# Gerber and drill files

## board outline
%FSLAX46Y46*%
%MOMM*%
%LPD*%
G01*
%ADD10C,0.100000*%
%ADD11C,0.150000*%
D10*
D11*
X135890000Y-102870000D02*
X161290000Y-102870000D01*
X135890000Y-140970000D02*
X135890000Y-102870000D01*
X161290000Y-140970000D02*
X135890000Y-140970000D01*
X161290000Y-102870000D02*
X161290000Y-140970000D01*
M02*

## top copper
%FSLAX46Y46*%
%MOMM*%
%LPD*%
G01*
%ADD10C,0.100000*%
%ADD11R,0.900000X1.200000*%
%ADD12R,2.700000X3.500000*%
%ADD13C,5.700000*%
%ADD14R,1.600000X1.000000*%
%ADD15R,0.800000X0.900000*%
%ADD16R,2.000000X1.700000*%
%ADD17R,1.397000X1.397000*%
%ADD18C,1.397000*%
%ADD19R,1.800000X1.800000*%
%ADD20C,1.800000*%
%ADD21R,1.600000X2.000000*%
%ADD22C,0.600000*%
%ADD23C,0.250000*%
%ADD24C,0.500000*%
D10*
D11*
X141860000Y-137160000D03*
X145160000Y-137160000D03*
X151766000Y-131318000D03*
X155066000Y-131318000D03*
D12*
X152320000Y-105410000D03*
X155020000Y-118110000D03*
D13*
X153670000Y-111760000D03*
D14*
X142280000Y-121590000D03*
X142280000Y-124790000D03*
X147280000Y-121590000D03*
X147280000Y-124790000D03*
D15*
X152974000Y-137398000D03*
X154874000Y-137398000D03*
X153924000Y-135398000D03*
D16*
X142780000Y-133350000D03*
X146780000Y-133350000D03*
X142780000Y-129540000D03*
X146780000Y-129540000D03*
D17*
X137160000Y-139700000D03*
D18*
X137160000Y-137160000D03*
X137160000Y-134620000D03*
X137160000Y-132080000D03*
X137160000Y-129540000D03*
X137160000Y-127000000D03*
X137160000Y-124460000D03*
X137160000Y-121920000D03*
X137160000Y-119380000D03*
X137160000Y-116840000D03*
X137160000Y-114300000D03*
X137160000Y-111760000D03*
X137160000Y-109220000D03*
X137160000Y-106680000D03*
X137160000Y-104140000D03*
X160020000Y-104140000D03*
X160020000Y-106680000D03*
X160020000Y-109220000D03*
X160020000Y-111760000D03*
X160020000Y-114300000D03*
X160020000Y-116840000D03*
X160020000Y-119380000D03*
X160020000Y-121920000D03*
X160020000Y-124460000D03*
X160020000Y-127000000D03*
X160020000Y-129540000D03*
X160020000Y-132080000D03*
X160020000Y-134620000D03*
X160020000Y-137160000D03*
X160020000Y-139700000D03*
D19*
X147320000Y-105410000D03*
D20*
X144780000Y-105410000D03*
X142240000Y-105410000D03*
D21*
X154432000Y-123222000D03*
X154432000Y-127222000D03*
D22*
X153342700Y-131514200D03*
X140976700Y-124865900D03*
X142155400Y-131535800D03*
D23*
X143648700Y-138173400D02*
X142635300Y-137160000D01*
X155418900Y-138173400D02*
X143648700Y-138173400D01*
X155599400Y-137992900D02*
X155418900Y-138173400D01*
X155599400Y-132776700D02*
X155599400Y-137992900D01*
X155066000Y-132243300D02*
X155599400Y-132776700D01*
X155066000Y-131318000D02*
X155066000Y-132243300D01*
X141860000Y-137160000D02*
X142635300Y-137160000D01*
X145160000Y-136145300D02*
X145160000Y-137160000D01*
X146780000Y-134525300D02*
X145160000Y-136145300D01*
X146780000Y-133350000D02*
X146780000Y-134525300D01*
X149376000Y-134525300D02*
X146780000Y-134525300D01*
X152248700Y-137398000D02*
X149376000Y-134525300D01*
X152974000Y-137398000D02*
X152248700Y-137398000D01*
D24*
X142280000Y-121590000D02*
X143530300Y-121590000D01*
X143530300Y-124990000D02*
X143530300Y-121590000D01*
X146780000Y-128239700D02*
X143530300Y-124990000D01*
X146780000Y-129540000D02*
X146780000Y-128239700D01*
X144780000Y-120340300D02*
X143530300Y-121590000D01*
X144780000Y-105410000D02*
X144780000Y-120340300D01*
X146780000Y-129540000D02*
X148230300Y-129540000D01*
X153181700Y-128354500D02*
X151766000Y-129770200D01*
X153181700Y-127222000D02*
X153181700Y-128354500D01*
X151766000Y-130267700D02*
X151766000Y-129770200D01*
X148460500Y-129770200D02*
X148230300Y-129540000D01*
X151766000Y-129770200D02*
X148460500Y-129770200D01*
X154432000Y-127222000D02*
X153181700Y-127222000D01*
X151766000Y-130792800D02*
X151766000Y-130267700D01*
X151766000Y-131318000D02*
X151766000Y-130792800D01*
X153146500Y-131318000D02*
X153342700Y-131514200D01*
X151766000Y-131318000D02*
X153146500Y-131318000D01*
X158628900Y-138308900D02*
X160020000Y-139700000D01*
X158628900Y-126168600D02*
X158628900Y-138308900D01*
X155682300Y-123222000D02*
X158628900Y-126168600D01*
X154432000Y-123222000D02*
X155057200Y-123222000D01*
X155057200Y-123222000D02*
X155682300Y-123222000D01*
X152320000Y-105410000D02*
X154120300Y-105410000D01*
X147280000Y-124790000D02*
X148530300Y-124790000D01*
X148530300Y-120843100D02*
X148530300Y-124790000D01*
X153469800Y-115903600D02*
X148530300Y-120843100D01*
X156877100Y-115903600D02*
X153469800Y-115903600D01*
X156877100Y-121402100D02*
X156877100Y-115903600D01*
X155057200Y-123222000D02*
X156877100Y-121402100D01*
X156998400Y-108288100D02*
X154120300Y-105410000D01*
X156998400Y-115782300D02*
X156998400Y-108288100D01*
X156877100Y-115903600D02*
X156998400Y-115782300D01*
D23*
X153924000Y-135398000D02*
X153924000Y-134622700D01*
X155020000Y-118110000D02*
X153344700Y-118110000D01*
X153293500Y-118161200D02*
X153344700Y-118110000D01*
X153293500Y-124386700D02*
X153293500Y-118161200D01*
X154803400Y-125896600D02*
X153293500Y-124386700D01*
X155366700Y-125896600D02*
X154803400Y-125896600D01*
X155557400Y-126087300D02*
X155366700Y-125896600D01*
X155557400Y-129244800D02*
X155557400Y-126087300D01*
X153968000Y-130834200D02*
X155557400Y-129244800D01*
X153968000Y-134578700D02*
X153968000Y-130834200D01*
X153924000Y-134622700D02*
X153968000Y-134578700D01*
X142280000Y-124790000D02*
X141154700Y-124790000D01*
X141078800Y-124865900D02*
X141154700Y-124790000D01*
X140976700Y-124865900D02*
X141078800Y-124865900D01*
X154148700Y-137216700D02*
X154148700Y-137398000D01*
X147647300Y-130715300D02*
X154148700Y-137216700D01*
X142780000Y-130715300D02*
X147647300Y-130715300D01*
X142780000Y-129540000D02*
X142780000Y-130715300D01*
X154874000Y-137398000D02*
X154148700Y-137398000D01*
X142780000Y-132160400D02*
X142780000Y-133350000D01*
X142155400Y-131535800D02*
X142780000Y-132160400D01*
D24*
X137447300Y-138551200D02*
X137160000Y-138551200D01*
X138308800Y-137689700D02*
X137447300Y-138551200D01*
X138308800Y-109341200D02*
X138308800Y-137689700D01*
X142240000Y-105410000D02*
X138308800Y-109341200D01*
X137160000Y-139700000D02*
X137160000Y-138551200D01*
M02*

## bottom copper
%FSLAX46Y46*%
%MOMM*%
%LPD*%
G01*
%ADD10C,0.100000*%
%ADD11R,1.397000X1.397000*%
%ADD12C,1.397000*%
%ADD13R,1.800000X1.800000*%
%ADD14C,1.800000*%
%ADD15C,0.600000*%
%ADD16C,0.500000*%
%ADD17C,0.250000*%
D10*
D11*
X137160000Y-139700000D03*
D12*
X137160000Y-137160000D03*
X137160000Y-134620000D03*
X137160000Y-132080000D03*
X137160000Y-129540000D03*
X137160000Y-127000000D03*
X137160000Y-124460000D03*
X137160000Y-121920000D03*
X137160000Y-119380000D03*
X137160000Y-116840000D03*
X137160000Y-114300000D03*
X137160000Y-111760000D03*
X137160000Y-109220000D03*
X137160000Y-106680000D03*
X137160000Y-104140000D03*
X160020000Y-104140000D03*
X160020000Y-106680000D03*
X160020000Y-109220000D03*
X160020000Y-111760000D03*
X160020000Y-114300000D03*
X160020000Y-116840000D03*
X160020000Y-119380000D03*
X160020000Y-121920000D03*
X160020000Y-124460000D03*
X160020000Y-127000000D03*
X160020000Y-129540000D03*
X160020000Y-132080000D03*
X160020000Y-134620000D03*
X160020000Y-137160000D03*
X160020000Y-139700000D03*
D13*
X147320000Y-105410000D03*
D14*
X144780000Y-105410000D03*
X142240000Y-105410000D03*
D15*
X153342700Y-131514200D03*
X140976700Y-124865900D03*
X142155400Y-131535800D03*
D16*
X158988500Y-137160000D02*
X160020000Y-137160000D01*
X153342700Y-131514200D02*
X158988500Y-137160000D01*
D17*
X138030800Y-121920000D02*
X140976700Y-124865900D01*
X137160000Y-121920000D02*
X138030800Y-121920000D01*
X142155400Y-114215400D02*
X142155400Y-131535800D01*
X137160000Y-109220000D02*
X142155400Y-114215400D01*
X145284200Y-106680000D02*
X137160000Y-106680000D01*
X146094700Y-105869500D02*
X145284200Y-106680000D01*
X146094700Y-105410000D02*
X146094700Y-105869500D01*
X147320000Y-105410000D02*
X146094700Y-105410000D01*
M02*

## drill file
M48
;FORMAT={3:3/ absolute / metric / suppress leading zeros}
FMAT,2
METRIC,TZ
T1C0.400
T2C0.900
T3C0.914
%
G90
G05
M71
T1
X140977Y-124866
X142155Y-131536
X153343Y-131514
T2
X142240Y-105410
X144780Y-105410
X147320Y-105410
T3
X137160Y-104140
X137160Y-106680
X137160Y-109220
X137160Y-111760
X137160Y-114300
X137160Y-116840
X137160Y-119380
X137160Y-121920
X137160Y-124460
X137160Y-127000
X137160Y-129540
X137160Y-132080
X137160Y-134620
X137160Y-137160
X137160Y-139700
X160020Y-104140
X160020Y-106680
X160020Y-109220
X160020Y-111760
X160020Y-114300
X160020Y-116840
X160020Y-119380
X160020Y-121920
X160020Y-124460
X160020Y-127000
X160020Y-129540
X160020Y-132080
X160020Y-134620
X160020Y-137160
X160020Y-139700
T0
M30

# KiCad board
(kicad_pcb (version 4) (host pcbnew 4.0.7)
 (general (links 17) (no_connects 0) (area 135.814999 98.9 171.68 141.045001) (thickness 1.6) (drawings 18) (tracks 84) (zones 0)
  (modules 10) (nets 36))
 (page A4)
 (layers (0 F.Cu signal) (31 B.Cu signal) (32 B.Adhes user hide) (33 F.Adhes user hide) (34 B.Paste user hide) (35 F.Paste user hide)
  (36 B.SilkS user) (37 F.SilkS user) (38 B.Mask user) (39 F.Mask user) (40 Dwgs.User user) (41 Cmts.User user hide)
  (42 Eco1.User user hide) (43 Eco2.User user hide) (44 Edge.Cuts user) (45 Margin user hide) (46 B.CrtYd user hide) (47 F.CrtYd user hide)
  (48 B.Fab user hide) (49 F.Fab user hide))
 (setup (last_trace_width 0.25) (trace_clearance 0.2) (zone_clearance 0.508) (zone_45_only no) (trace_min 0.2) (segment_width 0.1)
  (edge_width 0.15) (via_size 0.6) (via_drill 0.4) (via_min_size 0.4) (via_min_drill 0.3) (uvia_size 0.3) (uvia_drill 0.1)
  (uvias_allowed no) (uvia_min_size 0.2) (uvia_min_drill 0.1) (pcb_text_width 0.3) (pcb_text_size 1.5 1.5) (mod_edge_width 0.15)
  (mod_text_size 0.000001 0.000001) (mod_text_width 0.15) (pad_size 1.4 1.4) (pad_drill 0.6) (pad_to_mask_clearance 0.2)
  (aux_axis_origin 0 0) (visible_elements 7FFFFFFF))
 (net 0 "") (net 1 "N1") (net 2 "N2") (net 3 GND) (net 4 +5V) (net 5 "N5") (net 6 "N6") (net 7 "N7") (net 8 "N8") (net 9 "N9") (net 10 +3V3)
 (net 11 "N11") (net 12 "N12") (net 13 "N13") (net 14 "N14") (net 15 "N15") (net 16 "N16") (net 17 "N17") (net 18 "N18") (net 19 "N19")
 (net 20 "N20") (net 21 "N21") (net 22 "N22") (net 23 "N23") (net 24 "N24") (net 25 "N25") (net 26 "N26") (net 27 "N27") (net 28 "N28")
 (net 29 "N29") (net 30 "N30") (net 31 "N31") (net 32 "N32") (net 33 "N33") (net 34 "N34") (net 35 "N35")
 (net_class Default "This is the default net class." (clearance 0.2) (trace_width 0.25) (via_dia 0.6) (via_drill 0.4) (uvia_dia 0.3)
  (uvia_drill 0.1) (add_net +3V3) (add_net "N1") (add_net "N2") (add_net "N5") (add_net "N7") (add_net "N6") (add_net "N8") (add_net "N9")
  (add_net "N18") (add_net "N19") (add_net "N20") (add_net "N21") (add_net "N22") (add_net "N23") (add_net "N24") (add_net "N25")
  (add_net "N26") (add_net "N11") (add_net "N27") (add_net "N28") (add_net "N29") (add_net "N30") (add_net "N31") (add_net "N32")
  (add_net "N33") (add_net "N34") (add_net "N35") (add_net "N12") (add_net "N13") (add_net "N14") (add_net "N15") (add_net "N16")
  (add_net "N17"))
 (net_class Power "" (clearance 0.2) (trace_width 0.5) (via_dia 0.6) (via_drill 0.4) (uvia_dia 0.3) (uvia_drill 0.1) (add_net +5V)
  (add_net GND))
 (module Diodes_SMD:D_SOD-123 (layer F.Cu) (at 143.51 137.16)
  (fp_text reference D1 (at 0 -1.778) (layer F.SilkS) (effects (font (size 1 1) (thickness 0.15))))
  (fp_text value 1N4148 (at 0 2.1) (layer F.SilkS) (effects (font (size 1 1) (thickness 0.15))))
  (pad 1 smd rect (at -1.65 0) (size 0.9 1.2) (layers F.Cu F.Paste F.Mask) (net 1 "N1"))
  (pad 2 smd rect (at 1.65 0) (size 0.9 1.2) (layers F.Cu F.Paste F.Mask) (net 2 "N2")))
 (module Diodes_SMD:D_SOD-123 (layer F.Cu) (at 153.416 131.318)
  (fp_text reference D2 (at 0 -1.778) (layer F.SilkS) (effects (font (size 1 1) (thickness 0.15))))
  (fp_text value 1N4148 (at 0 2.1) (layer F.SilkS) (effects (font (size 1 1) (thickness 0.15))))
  (pad 1 smd rect (at -1.65 0) (size 0.9 1.2) (layers F.Cu F.Paste F.Mask) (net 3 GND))
  (pad 2 smd rect (at 1.65 0) (size 0.9 1.2) (layers F.Cu F.Paste F.Mask) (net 1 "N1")))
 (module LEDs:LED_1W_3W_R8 (layer F.Cu) (at 153.67 111.76 90)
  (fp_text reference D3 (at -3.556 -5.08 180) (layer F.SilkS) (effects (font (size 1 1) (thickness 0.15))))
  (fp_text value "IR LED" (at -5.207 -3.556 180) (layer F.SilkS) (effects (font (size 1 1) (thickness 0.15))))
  (pad 2 smd rect (at 6.35 -1.35 90) (size 3.5 2.7) (layers F.Cu F.Paste F.Mask) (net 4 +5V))
  (pad 1 smd rect (at -6.35 1.35 90) (size 3.5 2.7) (layers F.Cu F.Paste F.Mask) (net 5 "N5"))
  (pad 3 smd circle (at 0 0 90) (size 5.7 5.7) (layers F.Cu F.Paste F.Mask)))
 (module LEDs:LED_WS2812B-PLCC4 (layer F.Cu) (at 144.78 123.19 180)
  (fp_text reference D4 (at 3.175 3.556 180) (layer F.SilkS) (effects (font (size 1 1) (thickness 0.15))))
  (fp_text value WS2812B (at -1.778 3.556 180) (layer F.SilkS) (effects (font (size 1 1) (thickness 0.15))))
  (pad 3 smd rect (at 2.5 1.6 180) (size 1.6 1) (layers F.Cu F.Paste F.Mask) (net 3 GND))
  (pad 4 smd rect (at 2.5 -1.6 180) (size 1.6 1) (layers F.Cu F.Paste F.Mask) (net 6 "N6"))
  (pad 2 smd rect (at -2.5 1.6 180) (size 1.6 1) (layers F.Cu F.Paste F.Mask) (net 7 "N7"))
  (pad 1 smd rect (at -2.5 -1.6 180) (size 1.6 1) (layers F.Cu F.Paste F.Mask) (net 4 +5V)))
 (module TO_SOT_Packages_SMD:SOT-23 (layer F.Cu) (at 153.924 136.398 90)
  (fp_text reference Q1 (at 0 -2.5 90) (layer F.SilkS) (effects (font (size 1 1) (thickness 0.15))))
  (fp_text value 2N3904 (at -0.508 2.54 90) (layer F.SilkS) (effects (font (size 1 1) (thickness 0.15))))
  (pad 1 smd rect (at -1 -0.95 90) (size 0.9 0.8) (layers F.Cu F.Paste F.Mask) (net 2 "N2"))
  (pad 2 smd rect (at -1 0.95 90) (size 0.9 0.8) (layers F.Cu F.Paste F.Mask) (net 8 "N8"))
  (pad 3 smd rect (at 1 0 90) (size 0.9 0.8) (layers F.Cu F.Paste F.Mask) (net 5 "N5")))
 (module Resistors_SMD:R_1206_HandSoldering (layer F.Cu) (at 144.78 133.35)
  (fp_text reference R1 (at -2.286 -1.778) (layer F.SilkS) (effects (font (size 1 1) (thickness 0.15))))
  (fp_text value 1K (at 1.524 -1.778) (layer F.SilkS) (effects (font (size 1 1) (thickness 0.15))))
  (pad 1 smd rect (at -2 0) (size 2 1.7) (layers F.Cu F.Paste F.Mask) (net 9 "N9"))
  (pad 2 smd rect (at 2 0) (size 2 1.7) (layers F.Cu F.Paste F.Mask) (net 2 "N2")))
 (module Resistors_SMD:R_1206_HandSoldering (layer F.Cu) (at 144.78 129.54)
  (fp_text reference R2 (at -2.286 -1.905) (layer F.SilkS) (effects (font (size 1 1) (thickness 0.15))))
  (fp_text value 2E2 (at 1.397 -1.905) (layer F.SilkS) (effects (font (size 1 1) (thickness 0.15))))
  (pad 1 smd rect (at -2 0) (size 2 1.7) (layers F.Cu F.Paste F.Mask) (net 8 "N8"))
  (pad 2 smd rect (at 2 0) (size 2 1.7) (layers F.Cu F.Paste F.Mask) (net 3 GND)))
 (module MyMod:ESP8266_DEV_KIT (layer B.Cu) (at 148.59 139.7)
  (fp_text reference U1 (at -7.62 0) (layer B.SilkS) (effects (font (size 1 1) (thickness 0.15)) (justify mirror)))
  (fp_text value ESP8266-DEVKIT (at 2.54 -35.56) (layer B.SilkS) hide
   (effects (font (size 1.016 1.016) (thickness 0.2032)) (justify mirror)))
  (pad 1 thru_hole rect (at -11.43 0) (size 1.397 1.397) (drill 0.9144) (layers *.Cu *.Mask B.SilkS) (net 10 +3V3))
  (pad 2 thru_hole circle (at -11.43 -2.54) (size 1.397 1.397) (drill 0.9144) (layers *.Cu *.Mask B.SilkS) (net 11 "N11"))
  (pad 3 thru_hole circle (at -11.43 -5.08) (size 1.397 1.397) (drill 0.9144) (layers *.Cu *.Mask B.SilkS) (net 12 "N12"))
  (pad 4 thru_hole circle (at -11.43 -7.62) (size 1.397 1.397) (drill 0.9144) (layers *.Cu *.Mask B.SilkS) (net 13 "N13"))
  (pad 5 thru_hole circle (at -11.43 -10.16) (size 1.397 1.397) (drill 0.9144) (layers *.Cu *.Mask B.SilkS) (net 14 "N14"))
  (pad 6 thru_hole circle (at -11.43 -12.7) (size 1.397 1.397) (drill 0.9144) (layers *.Cu *.Mask B.SilkS) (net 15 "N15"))
  (pad 7 thru_hole circle (at -11.43 -15.24) (size 1.397 1.397) (drill 0.9144) (layers *.Cu *.Mask B.SilkS) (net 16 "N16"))
  (pad 8 thru_hole circle (at -11.43 -17.78) (size 1.397 1.397) (drill 0.9144) (layers *.Cu *.Mask B.SilkS) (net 6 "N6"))
  (pad 9 thru_hole circle (at -11.43 -20.32) (size 1.397 1.397) (drill 0.9144) (layers *.Cu *.Mask B.SilkS) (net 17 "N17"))
  (pad 10 thru_hole circle (at -11.43 -22.86) (size 1.397 1.397) (drill 0.9144) (layers *.Cu *.Mask B.SilkS) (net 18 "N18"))
  (pad 11 thru_hole circle (at -11.43 -25.4) (size 1.397 1.397) (drill 0.9144) (layers *.Cu *.Mask B.SilkS) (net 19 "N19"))
  (pad 12 thru_hole circle (at -11.43 -27.94) (size 1.397 1.397) (drill 0.9144) (layers *.Cu *.Mask B.SilkS) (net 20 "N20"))
  (pad 13 thru_hole circle (at -11.43 -30.48) (size 1.397 1.397) (drill 0.9144) (layers *.Cu *.Mask B.SilkS) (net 9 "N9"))
  (pad 14 thru_hole circle (at -11.43 -33.02) (size 1.397 1.397) (drill 0.9144) (layers *.Cu *.Mask B.SilkS) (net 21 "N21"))
  (pad 15 thru_hole circle (at -11.43 -35.56) (size 1.397 1.397) (drill 0.9144) (layers *.Cu *.Mask B.SilkS) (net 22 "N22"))
  (pad 16 thru_hole circle (at 11.43 -35.56) (size 1.397 1.397) (drill 0.9144) (layers *.Cu *.Mask B.SilkS) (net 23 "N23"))
  (pad 17 thru_hole circle (at 11.43 -33.02) (size 1.397 1.397) (drill 0.9144) (layers *.Cu *.Mask B.SilkS) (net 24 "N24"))
  (pad 18 thru_hole circle (at 11.43 -30.48) (size 1.397 1.397) (drill 0.9144) (layers *.Cu *.Mask B.SilkS) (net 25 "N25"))
  (pad 19 thru_hole circle (at 11.43 -27.94) (size 1.397 1.397) (drill 0.9144) (layers *.Cu *.Mask B.SilkS) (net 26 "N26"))
  (pad 20 thru_hole circle (at 11.43 -25.4) (size 1.397 1.397) (drill 0.9144) (layers *.Cu *.Mask B.SilkS) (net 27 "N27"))
  (pad 21 thru_hole circle (at 11.43 -22.86) (size 1.397 1.397) (drill 0.9144) (layers *.Cu *.Mask B.SilkS) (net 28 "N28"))
  (pad 22 thru_hole circle (at 11.43 -20.32) (size 1.397 1.397) (drill 0.9144) (layers *.Cu *.Mask B.SilkS) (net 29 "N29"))
  (pad 23 thru_hole circle (at 11.43 -17.78) (size 1.397 1.397) (drill 0.9144) (layers *.Cu *.Mask B.SilkS) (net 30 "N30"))
  (pad 24 thru_hole circle (at 11.43 -15.24) (size 1.397 1.397) (drill 0.9144) (layers *.Cu *.Mask B.SilkS) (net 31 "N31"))
  (pad 25 thru_hole circle (at 11.43 -12.7) (size 1.397 1.397) (drill 0.9144) (layers *.Cu *.Mask B.SilkS) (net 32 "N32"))
  (pad 26 thru_hole circle (at 11.43 -10.16) (size 1.397 1.397) (drill 0.9144) (layers *.Cu *.Mask B.SilkS) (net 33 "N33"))
  (pad 27 thru_hole circle (at 11.43 -7.62) (size 1.397 1.397) (drill 0.9144) (layers *.Cu *.Mask B.SilkS) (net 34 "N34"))
  (pad 28 thru_hole circle (at 11.43 -5.08) (size 1.397 1.397) (drill 0.9144) (layers *.Cu *.Mask B.SilkS) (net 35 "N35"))
  (pad 29 thru_hole circle (at 11.43 -2.54) (size 1.397 1.397) (drill 0.9144) (layers *.Cu *.Mask B.SilkS) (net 3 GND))
  (pad 30 thru_hole circle (at 11.43 0) (size 1.397 1.397) (drill 0.9144) (layers *.Cu *.Mask B.SilkS) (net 4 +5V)))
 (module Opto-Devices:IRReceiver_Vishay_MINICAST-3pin (layer F.Cu) (at 147.32 105.41 180)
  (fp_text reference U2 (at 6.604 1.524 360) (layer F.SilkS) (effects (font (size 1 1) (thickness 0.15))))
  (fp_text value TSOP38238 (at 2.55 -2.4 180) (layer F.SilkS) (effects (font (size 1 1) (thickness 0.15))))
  (pad 1 thru_hole rect (at 0 0 180) (size 1.8 1.8) (drill 0.9) (layers *.Cu *.Mask) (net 21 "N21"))
  (pad 2 thru_hole circle (at 2.54 0 180) (size 1.8 1.8) (drill 0.9) (layers *.Cu *.Mask) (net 3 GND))
  (pad 3 thru_hole circle (at 5.08 0 180) (size 1.8 1.8) (drill 0.9) (layers *.Cu *.Mask) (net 10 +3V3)))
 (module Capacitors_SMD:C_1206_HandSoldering (layer F.Cu) (at 154.432 125.222 270)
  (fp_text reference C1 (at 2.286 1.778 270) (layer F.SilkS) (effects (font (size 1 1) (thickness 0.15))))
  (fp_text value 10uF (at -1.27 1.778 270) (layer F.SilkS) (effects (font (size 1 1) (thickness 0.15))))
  (pad 1 smd rect (at -2 0 270) (size 2 1.6) (layers F.Cu F.Paste F.Mask) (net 4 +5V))
  (pad 2 smd rect (at 2 0 270) (size 2 1.6) (layers F.Cu F.Paste F.Mask) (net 3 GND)))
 (gr_line (start 135.89 102.87) (end 161.29 102.87) (angle 90) (layer Edge.Cuts) (width 0.15))
 (gr_line (start 135.89 140.97) (end 135.89 102.87) (angle 90) (layer Edge.Cuts) (width 0.15))
 (gr_line (start 161.29 140.97) (end 135.89 140.97) (angle 90) (layer Edge.Cuts) (width 0.15))
 (gr_line (start 161.29 102.87) (end 161.29 140.97) (angle 90) (layer Edge.Cuts) (width 0.15))
 (segment (start 143.6487 138.1734) (end 142.6353 137.16) (width 0.25) (layer F.Cu) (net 1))
 (segment (start 155.4189 138.1734) (end 143.6487 138.1734) (width 0.25) (layer F.Cu) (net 1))
 (segment (start 155.5994 137.9929) (end 155.4189 138.1734) (width 0.25) (layer F.Cu) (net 1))
 (segment (start 155.5994 132.7767) (end 155.5994 137.9929) (width 0.25) (layer F.Cu) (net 1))
 (segment (start 155.066 132.2433) (end 155.5994 132.7767) (width 0.25) (layer F.Cu) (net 1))
 (segment (start 155.066 131.318) (end 155.066 132.2433) (width 0.25) (layer F.Cu) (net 1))
 (segment (start 141.86 137.16) (end 142.6353 137.16) (width 0.25) (layer F.Cu) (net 1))
 (segment (start 145.16 136.1453) (end 145.16 137.16) (width 0.25) (layer F.Cu) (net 2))
 (segment (start 146.78 134.5253) (end 145.16 136.1453) (width 0.25) (layer F.Cu) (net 2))
 (segment (start 146.78 133.35) (end 146.78 134.5253) (width 0.25) (layer F.Cu) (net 2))
 (segment (start 149.376 134.5253) (end 146.78 134.5253) (width 0.25) (layer F.Cu) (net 2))
 (segment (start 152.2487 137.398) (end 149.376 134.5253) (width 0.25) (layer F.Cu) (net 2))
 (segment (start 152.974 137.398) (end 152.2487 137.398) (width 0.25) (layer F.Cu) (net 2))
 (via (at 153.3427 131.5142) (size 0.6) (layers F.Cu B.Cu) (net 3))
 (segment (start 142.28 121.59) (end 143.5303 121.59) (width 0.5) (layer F.Cu) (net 3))
 (segment (start 143.5303 124.99) (end 143.5303 121.59) (width 0.5) (layer F.Cu) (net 3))
 (segment (start 146.78 128.2397) (end 143.5303 124.99) (width 0.5) (layer F.Cu) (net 3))
 (segment (start 146.78 129.54) (end 146.78 128.2397) (width 0.5) (layer F.Cu) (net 3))
 (segment (start 144.78 120.3403) (end 143.5303 121.59) (width 0.5) (layer F.Cu) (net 3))
 (segment (start 144.78 105.41) (end 144.78 120.3403) (width 0.5) (layer F.Cu) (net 3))
 (segment (start 146.78 129.54) (end 148.2303 129.54) (width 0.5) (layer F.Cu) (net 3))
 (segment (start 153.1817 128.3545) (end 151.766 129.7702) (width 0.5) (layer F.Cu) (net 3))
 (segment (start 153.1817 127.222) (end 153.1817 128.3545) (width 0.5) (layer F.Cu) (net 3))
 (segment (start 151.766 130.2677) (end 151.766 129.7702) (width 0.5) (layer F.Cu) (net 3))
 (segment (start 148.4605 129.7702) (end 148.2303 129.54) (width 0.5) (layer F.Cu) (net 3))
 (segment (start 151.766 129.7702) (end 148.4605 129.7702) (width 0.5) (layer F.Cu) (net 3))
 (segment (start 154.432 127.222) (end 153.1817 127.222) (width 0.5) (layer F.Cu) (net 3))
 (segment (start 151.766 130.7928) (end 151.766 130.2677) (width 0.5) (layer F.Cu) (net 3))
 (segment (start 158.9885 137.16) (end 160.02 137.16) (width 0.5) (layer B.Cu) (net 3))
 (segment (start 153.3427 131.5142) (end 158.9885 137.16) (width 0.5) (layer B.Cu) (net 3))
 (segment (start 151.766 131.318) (end 151.766 130.7928) (width 0.5) (layer F.Cu) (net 3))
 (segment (start 153.1465 131.318) (end 153.3427 131.5142) (width 0.5) (layer F.Cu) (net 3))
 (segment (start 151.766 131.318) (end 153.1465 131.318) (width 0.5) (layer F.Cu) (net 3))
 (segment (start 158.6289 138.3089) (end 160.02 139.7) (width 0.5) (layer F.Cu) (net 4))
 (segment (start 158.6289 126.1686) (end 158.6289 138.3089) (width 0.5) (layer F.Cu) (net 4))
 (segment (start 155.6823 123.222) (end 158.6289 126.1686) (width 0.5) (layer F.Cu) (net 4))
 (segment (start 154.432 123.222) (end 155.0572 123.222) (width 0.5) (layer F.Cu) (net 4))
 (segment (start 155.0572 123.222) (end 155.6823 123.222) (width 0.5) (layer F.Cu) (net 4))
 (segment (start 152.32 105.41) (end 154.1203 105.41) (width 0.5) (layer F.Cu) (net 4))
 (segment (start 147.28 124.79) (end 148.5303 124.79) (width 0.5) (layer F.Cu) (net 4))
 (segment (start 148.5303 120.8431) (end 148.5303 124.79) (width 0.5) (layer F.Cu) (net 4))
 (segment (start 153.4698 115.9036) (end 148.5303 120.8431) (width 0.5) (layer F.Cu) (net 4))
 (segment (start 156.8771 115.9036) (end 153.4698 115.9036) (width 0.5) (layer F.Cu) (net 4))
 (segment (start 156.8771 121.4021) (end 156.8771 115.9036) (width 0.5) (layer F.Cu) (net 4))
 (segment (start 155.0572 123.222) (end 156.8771 121.4021) (width 0.5) (layer F.Cu) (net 4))
 (segment (start 156.9984 108.2881) (end 154.1203 105.41) (width 0.5) (layer F.Cu) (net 4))
 (segment (start 156.9984 115.7823) (end 156.9984 108.2881) (width 0.5) (layer F.Cu) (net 4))
 (segment (start 156.8771 115.9036) (end 156.9984 115.7823) (width 0.5) (layer F.Cu) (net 4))
 (segment (start 153.924 135.398) (end 153.924 134.6227) (width 0.25) (layer F.Cu) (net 5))
 (segment (start 155.02 118.11) (end 153.3447 118.11) (width 0.25) (layer F.Cu) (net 5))
 (segment (start 153.2935 118.1612) (end 153.3447 118.11) (width 0.25) (layer F.Cu) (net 5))
 (segment (start 153.2935 124.3867) (end 153.2935 118.1612) (width 0.25) (layer F.Cu) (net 5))
 (segment (start 154.8034 125.8966) (end 153.2935 124.3867) (width 0.25) (layer F.Cu) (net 5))
 (segment (start 155.3667 125.8966) (end 154.8034 125.8966) (width 0.25) (layer F.Cu) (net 5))
 (segment (start 155.5574 126.0873) (end 155.3667 125.8966) (width 0.25) (layer F.Cu) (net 5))
 (segment (start 155.5574 129.2448) (end 155.5574 126.0873) (width 0.25) (layer F.Cu) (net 5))
 (segment (start 153.968 130.8342) (end 155.5574 129.2448) (width 0.25) (layer F.Cu) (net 5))
 (segment (start 153.968 134.5787) (end 153.968 130.8342) (width 0.25) (layer F.Cu) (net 5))
 (segment (start 153.924 134.6227) (end 153.968 134.5787) (width 0.25) (layer F.Cu) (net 5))
 (via (at 140.9767 124.8659) (size 0.6) (layers F.Cu B.Cu) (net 6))
 (segment (start 142.28 124.79) (end 141.1547 124.79) (width 0.25) (layer F.Cu) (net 6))
 (segment (start 138.0308 121.92) (end 140.9767 124.8659) (width 0.25) (layer B.Cu) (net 6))
 (segment (start 137.16 121.92) (end 138.0308 121.92) (width 0.25) (layer B.Cu) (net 6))
 (segment (start 141.0788 124.8659) (end 141.1547 124.79) (width 0.25) (layer F.Cu) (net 6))
 (segment (start 140.9767 124.8659) (end 141.0788 124.8659) (width 0.25) (layer F.Cu) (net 6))
 (segment (start 154.1487 137.2167) (end 154.1487 137.398) (width 0.25) (layer F.Cu) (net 8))
 (segment (start 147.6473 130.7153) (end 154.1487 137.2167) (width 0.25) (layer F.Cu) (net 8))
 (segment (start 142.78 130.7153) (end 147.6473 130.7153) (width 0.25) (layer F.Cu) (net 8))
 (segment (start 142.78 129.54) (end 142.78 130.7153) (width 0.25) (layer F.Cu) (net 8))
 (segment (start 154.874 137.398) (end 154.1487 137.398) (width 0.25) (layer F.Cu) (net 8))
 (via (at 142.1554 131.5358) (size 0.6) (layers F.Cu B.Cu) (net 9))
 (segment (start 142.1554 114.2154) (end 142.1554 131.5358) (width 0.25) (layer B.Cu) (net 9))
 (segment (start 137.16 109.22) (end 142.1554 114.2154) (width 0.25) (layer B.Cu) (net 9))
 (segment (start 142.78 132.1604) (end 142.78 133.35) (width 0.25) (layer F.Cu) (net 9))
 (segment (start 142.1554 131.5358) (end 142.78 132.1604) (width 0.25) (layer F.Cu) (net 9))
 (segment (start 137.4473 138.5512) (end 137.16 138.5512) (width 0.5) (layer F.Cu) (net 10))
 (segment (start 138.3088 137.6897) (end 137.4473 138.5512) (width 0.5) (layer F.Cu) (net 10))
 (segment (start 138.3088 109.3412) (end 138.3088 137.6897) (width 0.5) (layer F.Cu) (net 10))
 (segment (start 142.24 105.41) (end 138.3088 109.3412) (width 0.5) (layer F.Cu) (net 10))
 (segment (start 137.16 139.7) (end 137.16 138.5512) (width 0.5) (layer F.Cu) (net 10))
 (segment (start 145.2842 106.68) (end 137.16 106.68) (width 0.25) (layer B.Cu) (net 21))
 (segment (start 146.0947 105.8695) (end 145.2842 106.68) (width 0.25) (layer B.Cu) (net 21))
 (segment (start 146.0947 105.41) (end 146.0947 105.8695) (width 0.25) (layer B.Cu) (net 21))
 (segment (start 147.32 105.41) (end 146.0947 105.41) (width 0.25) (layer B.Cu) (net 21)))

